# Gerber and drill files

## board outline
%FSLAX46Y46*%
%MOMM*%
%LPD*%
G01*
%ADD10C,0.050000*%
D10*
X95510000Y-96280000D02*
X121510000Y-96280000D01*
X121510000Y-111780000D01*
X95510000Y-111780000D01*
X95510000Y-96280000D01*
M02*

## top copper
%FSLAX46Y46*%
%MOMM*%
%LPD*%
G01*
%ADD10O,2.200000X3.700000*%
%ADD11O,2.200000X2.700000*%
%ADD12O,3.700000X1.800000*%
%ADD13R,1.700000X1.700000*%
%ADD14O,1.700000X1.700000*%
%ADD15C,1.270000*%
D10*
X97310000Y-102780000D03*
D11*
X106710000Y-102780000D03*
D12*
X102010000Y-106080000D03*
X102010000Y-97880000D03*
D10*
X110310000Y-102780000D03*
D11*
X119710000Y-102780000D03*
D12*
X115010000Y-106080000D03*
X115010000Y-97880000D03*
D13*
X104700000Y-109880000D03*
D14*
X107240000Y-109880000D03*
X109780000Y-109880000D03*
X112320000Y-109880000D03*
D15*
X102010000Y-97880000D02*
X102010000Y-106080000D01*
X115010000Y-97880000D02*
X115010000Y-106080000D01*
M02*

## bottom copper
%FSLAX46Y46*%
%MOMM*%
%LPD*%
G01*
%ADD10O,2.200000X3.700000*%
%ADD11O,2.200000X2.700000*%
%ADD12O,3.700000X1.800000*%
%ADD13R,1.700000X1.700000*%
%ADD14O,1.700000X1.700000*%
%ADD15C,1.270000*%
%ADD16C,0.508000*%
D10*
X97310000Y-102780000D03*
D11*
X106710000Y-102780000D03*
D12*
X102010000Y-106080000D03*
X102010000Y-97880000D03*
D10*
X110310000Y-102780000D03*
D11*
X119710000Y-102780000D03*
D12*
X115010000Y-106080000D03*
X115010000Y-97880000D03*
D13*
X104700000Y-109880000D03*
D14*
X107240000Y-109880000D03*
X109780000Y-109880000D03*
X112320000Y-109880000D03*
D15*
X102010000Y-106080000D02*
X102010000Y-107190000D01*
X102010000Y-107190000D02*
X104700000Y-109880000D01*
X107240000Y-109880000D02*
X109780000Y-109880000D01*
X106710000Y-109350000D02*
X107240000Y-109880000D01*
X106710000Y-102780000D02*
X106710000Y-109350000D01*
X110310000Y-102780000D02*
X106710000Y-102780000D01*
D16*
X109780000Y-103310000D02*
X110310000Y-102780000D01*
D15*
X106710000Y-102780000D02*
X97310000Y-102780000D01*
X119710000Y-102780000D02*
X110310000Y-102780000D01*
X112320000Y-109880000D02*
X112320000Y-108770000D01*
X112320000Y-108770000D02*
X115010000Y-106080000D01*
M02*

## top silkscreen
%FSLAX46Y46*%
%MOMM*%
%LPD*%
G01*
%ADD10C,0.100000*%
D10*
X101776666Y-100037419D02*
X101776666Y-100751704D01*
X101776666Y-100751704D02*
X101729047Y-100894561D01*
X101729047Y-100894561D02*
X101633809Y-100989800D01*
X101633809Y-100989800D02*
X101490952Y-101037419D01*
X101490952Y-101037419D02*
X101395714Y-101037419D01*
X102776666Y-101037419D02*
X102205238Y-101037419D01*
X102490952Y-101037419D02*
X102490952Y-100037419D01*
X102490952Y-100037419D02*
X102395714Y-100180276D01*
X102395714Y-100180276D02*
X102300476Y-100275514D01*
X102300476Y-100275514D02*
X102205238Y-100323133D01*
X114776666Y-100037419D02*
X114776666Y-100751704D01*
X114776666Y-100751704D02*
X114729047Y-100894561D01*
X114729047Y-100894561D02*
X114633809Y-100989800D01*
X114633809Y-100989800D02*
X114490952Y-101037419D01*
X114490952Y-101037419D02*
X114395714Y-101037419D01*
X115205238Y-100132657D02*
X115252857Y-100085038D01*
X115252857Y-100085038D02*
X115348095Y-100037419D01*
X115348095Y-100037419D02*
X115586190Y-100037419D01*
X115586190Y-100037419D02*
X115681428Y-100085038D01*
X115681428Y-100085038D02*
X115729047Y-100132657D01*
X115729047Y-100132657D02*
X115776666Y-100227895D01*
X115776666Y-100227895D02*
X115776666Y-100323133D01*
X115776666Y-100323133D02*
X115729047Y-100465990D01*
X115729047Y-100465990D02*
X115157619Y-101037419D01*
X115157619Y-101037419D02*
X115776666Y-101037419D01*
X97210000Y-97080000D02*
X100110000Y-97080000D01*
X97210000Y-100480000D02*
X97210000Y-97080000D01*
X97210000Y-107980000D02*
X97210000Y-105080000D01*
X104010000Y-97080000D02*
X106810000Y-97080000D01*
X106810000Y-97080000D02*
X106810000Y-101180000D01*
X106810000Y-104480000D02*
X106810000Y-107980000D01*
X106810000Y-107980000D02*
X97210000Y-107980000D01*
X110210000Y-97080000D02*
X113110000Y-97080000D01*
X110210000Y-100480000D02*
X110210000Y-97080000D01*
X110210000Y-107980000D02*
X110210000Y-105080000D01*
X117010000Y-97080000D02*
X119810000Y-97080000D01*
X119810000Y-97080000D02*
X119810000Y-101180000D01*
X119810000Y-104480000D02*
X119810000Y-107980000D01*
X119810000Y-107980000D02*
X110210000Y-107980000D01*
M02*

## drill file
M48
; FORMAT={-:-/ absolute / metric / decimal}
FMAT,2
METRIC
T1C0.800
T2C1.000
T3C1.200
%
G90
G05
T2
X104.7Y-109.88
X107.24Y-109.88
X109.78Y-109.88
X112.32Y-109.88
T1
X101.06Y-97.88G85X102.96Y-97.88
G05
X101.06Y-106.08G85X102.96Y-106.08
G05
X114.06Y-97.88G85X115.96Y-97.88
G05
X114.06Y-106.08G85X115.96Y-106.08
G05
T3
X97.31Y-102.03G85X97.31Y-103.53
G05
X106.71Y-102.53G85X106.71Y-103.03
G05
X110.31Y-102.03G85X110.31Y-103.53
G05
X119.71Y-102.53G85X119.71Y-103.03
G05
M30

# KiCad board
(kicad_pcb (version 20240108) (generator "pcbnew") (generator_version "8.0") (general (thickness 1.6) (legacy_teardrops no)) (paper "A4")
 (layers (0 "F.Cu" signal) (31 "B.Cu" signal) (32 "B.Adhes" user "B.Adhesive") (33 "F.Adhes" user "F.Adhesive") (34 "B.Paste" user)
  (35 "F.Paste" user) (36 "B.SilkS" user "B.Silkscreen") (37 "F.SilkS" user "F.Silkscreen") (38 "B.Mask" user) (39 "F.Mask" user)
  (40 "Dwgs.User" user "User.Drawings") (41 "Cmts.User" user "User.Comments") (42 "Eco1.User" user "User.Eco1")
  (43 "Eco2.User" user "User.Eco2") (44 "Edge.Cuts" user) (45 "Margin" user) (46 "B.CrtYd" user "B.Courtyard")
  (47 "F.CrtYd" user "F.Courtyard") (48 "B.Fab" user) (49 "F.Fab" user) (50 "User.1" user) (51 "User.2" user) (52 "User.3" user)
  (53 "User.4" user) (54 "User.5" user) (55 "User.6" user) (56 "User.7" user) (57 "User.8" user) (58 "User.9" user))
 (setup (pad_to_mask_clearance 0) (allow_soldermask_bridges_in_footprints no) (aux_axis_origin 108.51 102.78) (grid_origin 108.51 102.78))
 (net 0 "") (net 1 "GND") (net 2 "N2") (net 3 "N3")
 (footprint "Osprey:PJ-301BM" (layer "F.Cu") (at 102.01 102.78)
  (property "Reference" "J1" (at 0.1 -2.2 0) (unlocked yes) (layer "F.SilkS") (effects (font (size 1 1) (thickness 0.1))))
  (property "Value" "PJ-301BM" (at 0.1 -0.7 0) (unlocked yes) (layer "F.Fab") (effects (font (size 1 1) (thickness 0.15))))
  (fp_line (start -4.8 -5.7) (end -1.9 -5.7) (stroke (width 0.1) (type default)) (layer "F.SilkS"))
  (fp_line (start -4.8 -2.3) (end -4.8 -5.7) (stroke (width 0.1) (type default)) (layer "F.SilkS"))
  (fp_line (start -4.8 5.2) (end -4.8 2.3) (stroke (width 0.1) (type default)) (layer "F.SilkS"))
  (fp_line (start 2 -5.7) (end 4.8 -5.7) (stroke (width 0.1) (type default)) (layer "F.SilkS"))
  (fp_line (start 4.8 -5.7) (end 4.8 -1.6) (stroke (width 0.1) (type default)) (layer "F.SilkS"))
  (fp_line (start 4.8 1.7) (end 4.8 5.2) (stroke (width 0.1) (type default)) (layer "F.SilkS"))
  (fp_line (start 4.8 5.2) (end -4.8 5.2) (stroke (width 0.1) (type default)) (layer "F.SilkS"))
  (pad "1" thru_hole oval (at -4.7 0) (size 2.2 3.7) (drill oval 1.2 2.7) (layers "*.Cu" "*.Mask") (remove_unused_layers no) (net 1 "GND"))
  (pad "1" thru_hole oval (at 4.7 0) (size 2.2 2.7) (drill oval 1.2 1.7) (layers "*.Cu" "*.Mask") (remove_unused_layers no) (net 1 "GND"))
  (pad "2" thru_hole oval (at 0 3.3) (size 3.7 1.8) (drill oval 2.7 0.8) (layers "*.Cu" "*.Mask") (remove_unused_layers no) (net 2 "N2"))
  (pad "3" thru_hole oval (at 0 -4.9) (size 3.7 1.8) (drill oval 2.7 0.8) (layers "*.Cu" "*.Mask") (remove_unused_layers no) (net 2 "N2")))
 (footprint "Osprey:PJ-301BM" (layer "F.Cu") (at 115.01 102.78)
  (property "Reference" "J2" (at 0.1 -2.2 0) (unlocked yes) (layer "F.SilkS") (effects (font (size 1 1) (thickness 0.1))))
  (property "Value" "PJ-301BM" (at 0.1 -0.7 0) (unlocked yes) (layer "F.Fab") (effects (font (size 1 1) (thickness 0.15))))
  (fp_line (start -4.8 -5.7) (end -1.9 -5.7) (stroke (width 0.1) (type default)) (layer "F.SilkS"))
  (fp_line (start -4.8 -2.3) (end -4.8 -5.7) (stroke (width 0.1) (type default)) (layer "F.SilkS"))
  (fp_line (start -4.8 5.2) (end -4.8 2.3) (stroke (width 0.1) (type default)) (layer "F.SilkS"))
  (fp_line (start 2 -5.7) (end 4.8 -5.7) (stroke (width 0.1) (type default)) (layer "F.SilkS"))
  (fp_line (start 4.8 -5.7) (end 4.8 -1.6) (stroke (width 0.1) (type default)) (layer "F.SilkS"))
  (fp_line (start 4.8 1.7) (end 4.8 5.2) (stroke (width 0.1) (type default)) (layer "F.SilkS"))
  (fp_line (start 4.8 5.2) (end -4.8 5.2) (stroke (width 0.1) (type default)) (layer "F.SilkS"))
  (pad "1" thru_hole oval (at -4.7 0) (size 2.2 3.7) (drill oval 1.2 2.7) (layers "*.Cu" "*.Mask") (remove_unused_layers no) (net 1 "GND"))
  (pad "1" thru_hole oval (at 4.7 0) (size 2.2 2.7) (drill oval 1.2 1.7) (layers "*.Cu" "*.Mask") (remove_unused_layers no) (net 1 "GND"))
  (pad "2" thru_hole oval (at 0 3.3) (size 3.7 1.8) (drill oval 2.7 0.8) (layers "*.Cu" "*.Mask") (remove_unused_layers no) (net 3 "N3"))
  (pad "3" thru_hole oval (at 0 -4.9) (size 3.7 1.8) (drill oval 2.7 0.8) (layers "*.Cu" "*.Mask") (remove_unused_layers no) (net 3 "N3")))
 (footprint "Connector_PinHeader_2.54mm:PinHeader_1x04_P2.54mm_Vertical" (layer "B.Cu") (at 104.7 109.88 -90)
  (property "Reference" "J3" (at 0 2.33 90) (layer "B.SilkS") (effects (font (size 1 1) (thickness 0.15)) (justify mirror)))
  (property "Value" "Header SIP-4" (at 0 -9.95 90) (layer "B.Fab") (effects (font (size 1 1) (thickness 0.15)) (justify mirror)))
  (pad "1" thru_hole rect (at 0 0 270) (size 1.7 1.7) (drill 1) (layers "*.Cu" "*.Mask") (remove_unused_layers no) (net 2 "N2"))
  (pad "2" thru_hole oval (at 0 -2.54 270) (size 1.7 1.7) (drill 1) (layers "*.Cu" "*.Mask") (remove_unused_layers no) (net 1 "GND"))
  (pad "3" thru_hole oval (at 0 -5.08 270) (size 1.7 1.7) (drill 1) (layers "*.Cu" "*.Mask") (remove_unused_layers no) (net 1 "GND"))
  (pad "4" thru_hole oval (at 0 -7.62 270) (size 1.7 1.7) (drill 1) (layers "*.Cu" "*.Mask") (remove_unused_layers no) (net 3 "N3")))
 (gr_rect (start 95.51 96.28) (end 121.51 111.78) (stroke (width 0.05) (type default)) (fill none) (layer "Edge.Cuts"))
 (segment (start 102.01 97.88) (end 102.01 106.08) (width 1.27) (layer "F.Cu") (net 2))
 (segment (start 102.01 106.08) (end 102.01 107.19) (width 1.27) (layer "B.Cu") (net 2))
 (segment (start 102.01 107.19) (end 104.7 109.88) (width 1.27) (layer "B.Cu") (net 2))
 (segment (start 107.24 109.88) (end 109.78 109.88) (width 1.27) (layer "B.Cu") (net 1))
 (segment (start 106.71 109.35) (end 107.24 109.88) (width 1.27) (layer "B.Cu") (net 1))
 (segment (start 106.71 102.78) (end 106.71 109.35) (width 1.27) (layer "B.Cu") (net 1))
 (segment (start 110.31 102.78) (end 106.71 102.78) (width 1.27) (layer "B.Cu") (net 1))
 (segment (start 109.78 103.31) (end 110.31 102.78) (width 0.508) (layer "B.Cu") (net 1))
 (segment (start 106.71 102.78) (end 97.31 102.78) (width 1.27) (layer "B.Cu") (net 1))
 (segment (start 119.71 102.78) (end 110.31 102.78) (width 1.27) (layer "B.Cu") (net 1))
 (segment (start 115.01 97.88) (end 115.01 106.08) (width 1.27) (layer "F.Cu") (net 3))
 (segment (start 112.32 109.88) (end 112.32 108.77) (width 1.27) (layer "B.Cu") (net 3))
 (segment (start 112.32 108.77) (end 115.01 106.08) (width 1.27) (layer "B.Cu") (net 3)))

